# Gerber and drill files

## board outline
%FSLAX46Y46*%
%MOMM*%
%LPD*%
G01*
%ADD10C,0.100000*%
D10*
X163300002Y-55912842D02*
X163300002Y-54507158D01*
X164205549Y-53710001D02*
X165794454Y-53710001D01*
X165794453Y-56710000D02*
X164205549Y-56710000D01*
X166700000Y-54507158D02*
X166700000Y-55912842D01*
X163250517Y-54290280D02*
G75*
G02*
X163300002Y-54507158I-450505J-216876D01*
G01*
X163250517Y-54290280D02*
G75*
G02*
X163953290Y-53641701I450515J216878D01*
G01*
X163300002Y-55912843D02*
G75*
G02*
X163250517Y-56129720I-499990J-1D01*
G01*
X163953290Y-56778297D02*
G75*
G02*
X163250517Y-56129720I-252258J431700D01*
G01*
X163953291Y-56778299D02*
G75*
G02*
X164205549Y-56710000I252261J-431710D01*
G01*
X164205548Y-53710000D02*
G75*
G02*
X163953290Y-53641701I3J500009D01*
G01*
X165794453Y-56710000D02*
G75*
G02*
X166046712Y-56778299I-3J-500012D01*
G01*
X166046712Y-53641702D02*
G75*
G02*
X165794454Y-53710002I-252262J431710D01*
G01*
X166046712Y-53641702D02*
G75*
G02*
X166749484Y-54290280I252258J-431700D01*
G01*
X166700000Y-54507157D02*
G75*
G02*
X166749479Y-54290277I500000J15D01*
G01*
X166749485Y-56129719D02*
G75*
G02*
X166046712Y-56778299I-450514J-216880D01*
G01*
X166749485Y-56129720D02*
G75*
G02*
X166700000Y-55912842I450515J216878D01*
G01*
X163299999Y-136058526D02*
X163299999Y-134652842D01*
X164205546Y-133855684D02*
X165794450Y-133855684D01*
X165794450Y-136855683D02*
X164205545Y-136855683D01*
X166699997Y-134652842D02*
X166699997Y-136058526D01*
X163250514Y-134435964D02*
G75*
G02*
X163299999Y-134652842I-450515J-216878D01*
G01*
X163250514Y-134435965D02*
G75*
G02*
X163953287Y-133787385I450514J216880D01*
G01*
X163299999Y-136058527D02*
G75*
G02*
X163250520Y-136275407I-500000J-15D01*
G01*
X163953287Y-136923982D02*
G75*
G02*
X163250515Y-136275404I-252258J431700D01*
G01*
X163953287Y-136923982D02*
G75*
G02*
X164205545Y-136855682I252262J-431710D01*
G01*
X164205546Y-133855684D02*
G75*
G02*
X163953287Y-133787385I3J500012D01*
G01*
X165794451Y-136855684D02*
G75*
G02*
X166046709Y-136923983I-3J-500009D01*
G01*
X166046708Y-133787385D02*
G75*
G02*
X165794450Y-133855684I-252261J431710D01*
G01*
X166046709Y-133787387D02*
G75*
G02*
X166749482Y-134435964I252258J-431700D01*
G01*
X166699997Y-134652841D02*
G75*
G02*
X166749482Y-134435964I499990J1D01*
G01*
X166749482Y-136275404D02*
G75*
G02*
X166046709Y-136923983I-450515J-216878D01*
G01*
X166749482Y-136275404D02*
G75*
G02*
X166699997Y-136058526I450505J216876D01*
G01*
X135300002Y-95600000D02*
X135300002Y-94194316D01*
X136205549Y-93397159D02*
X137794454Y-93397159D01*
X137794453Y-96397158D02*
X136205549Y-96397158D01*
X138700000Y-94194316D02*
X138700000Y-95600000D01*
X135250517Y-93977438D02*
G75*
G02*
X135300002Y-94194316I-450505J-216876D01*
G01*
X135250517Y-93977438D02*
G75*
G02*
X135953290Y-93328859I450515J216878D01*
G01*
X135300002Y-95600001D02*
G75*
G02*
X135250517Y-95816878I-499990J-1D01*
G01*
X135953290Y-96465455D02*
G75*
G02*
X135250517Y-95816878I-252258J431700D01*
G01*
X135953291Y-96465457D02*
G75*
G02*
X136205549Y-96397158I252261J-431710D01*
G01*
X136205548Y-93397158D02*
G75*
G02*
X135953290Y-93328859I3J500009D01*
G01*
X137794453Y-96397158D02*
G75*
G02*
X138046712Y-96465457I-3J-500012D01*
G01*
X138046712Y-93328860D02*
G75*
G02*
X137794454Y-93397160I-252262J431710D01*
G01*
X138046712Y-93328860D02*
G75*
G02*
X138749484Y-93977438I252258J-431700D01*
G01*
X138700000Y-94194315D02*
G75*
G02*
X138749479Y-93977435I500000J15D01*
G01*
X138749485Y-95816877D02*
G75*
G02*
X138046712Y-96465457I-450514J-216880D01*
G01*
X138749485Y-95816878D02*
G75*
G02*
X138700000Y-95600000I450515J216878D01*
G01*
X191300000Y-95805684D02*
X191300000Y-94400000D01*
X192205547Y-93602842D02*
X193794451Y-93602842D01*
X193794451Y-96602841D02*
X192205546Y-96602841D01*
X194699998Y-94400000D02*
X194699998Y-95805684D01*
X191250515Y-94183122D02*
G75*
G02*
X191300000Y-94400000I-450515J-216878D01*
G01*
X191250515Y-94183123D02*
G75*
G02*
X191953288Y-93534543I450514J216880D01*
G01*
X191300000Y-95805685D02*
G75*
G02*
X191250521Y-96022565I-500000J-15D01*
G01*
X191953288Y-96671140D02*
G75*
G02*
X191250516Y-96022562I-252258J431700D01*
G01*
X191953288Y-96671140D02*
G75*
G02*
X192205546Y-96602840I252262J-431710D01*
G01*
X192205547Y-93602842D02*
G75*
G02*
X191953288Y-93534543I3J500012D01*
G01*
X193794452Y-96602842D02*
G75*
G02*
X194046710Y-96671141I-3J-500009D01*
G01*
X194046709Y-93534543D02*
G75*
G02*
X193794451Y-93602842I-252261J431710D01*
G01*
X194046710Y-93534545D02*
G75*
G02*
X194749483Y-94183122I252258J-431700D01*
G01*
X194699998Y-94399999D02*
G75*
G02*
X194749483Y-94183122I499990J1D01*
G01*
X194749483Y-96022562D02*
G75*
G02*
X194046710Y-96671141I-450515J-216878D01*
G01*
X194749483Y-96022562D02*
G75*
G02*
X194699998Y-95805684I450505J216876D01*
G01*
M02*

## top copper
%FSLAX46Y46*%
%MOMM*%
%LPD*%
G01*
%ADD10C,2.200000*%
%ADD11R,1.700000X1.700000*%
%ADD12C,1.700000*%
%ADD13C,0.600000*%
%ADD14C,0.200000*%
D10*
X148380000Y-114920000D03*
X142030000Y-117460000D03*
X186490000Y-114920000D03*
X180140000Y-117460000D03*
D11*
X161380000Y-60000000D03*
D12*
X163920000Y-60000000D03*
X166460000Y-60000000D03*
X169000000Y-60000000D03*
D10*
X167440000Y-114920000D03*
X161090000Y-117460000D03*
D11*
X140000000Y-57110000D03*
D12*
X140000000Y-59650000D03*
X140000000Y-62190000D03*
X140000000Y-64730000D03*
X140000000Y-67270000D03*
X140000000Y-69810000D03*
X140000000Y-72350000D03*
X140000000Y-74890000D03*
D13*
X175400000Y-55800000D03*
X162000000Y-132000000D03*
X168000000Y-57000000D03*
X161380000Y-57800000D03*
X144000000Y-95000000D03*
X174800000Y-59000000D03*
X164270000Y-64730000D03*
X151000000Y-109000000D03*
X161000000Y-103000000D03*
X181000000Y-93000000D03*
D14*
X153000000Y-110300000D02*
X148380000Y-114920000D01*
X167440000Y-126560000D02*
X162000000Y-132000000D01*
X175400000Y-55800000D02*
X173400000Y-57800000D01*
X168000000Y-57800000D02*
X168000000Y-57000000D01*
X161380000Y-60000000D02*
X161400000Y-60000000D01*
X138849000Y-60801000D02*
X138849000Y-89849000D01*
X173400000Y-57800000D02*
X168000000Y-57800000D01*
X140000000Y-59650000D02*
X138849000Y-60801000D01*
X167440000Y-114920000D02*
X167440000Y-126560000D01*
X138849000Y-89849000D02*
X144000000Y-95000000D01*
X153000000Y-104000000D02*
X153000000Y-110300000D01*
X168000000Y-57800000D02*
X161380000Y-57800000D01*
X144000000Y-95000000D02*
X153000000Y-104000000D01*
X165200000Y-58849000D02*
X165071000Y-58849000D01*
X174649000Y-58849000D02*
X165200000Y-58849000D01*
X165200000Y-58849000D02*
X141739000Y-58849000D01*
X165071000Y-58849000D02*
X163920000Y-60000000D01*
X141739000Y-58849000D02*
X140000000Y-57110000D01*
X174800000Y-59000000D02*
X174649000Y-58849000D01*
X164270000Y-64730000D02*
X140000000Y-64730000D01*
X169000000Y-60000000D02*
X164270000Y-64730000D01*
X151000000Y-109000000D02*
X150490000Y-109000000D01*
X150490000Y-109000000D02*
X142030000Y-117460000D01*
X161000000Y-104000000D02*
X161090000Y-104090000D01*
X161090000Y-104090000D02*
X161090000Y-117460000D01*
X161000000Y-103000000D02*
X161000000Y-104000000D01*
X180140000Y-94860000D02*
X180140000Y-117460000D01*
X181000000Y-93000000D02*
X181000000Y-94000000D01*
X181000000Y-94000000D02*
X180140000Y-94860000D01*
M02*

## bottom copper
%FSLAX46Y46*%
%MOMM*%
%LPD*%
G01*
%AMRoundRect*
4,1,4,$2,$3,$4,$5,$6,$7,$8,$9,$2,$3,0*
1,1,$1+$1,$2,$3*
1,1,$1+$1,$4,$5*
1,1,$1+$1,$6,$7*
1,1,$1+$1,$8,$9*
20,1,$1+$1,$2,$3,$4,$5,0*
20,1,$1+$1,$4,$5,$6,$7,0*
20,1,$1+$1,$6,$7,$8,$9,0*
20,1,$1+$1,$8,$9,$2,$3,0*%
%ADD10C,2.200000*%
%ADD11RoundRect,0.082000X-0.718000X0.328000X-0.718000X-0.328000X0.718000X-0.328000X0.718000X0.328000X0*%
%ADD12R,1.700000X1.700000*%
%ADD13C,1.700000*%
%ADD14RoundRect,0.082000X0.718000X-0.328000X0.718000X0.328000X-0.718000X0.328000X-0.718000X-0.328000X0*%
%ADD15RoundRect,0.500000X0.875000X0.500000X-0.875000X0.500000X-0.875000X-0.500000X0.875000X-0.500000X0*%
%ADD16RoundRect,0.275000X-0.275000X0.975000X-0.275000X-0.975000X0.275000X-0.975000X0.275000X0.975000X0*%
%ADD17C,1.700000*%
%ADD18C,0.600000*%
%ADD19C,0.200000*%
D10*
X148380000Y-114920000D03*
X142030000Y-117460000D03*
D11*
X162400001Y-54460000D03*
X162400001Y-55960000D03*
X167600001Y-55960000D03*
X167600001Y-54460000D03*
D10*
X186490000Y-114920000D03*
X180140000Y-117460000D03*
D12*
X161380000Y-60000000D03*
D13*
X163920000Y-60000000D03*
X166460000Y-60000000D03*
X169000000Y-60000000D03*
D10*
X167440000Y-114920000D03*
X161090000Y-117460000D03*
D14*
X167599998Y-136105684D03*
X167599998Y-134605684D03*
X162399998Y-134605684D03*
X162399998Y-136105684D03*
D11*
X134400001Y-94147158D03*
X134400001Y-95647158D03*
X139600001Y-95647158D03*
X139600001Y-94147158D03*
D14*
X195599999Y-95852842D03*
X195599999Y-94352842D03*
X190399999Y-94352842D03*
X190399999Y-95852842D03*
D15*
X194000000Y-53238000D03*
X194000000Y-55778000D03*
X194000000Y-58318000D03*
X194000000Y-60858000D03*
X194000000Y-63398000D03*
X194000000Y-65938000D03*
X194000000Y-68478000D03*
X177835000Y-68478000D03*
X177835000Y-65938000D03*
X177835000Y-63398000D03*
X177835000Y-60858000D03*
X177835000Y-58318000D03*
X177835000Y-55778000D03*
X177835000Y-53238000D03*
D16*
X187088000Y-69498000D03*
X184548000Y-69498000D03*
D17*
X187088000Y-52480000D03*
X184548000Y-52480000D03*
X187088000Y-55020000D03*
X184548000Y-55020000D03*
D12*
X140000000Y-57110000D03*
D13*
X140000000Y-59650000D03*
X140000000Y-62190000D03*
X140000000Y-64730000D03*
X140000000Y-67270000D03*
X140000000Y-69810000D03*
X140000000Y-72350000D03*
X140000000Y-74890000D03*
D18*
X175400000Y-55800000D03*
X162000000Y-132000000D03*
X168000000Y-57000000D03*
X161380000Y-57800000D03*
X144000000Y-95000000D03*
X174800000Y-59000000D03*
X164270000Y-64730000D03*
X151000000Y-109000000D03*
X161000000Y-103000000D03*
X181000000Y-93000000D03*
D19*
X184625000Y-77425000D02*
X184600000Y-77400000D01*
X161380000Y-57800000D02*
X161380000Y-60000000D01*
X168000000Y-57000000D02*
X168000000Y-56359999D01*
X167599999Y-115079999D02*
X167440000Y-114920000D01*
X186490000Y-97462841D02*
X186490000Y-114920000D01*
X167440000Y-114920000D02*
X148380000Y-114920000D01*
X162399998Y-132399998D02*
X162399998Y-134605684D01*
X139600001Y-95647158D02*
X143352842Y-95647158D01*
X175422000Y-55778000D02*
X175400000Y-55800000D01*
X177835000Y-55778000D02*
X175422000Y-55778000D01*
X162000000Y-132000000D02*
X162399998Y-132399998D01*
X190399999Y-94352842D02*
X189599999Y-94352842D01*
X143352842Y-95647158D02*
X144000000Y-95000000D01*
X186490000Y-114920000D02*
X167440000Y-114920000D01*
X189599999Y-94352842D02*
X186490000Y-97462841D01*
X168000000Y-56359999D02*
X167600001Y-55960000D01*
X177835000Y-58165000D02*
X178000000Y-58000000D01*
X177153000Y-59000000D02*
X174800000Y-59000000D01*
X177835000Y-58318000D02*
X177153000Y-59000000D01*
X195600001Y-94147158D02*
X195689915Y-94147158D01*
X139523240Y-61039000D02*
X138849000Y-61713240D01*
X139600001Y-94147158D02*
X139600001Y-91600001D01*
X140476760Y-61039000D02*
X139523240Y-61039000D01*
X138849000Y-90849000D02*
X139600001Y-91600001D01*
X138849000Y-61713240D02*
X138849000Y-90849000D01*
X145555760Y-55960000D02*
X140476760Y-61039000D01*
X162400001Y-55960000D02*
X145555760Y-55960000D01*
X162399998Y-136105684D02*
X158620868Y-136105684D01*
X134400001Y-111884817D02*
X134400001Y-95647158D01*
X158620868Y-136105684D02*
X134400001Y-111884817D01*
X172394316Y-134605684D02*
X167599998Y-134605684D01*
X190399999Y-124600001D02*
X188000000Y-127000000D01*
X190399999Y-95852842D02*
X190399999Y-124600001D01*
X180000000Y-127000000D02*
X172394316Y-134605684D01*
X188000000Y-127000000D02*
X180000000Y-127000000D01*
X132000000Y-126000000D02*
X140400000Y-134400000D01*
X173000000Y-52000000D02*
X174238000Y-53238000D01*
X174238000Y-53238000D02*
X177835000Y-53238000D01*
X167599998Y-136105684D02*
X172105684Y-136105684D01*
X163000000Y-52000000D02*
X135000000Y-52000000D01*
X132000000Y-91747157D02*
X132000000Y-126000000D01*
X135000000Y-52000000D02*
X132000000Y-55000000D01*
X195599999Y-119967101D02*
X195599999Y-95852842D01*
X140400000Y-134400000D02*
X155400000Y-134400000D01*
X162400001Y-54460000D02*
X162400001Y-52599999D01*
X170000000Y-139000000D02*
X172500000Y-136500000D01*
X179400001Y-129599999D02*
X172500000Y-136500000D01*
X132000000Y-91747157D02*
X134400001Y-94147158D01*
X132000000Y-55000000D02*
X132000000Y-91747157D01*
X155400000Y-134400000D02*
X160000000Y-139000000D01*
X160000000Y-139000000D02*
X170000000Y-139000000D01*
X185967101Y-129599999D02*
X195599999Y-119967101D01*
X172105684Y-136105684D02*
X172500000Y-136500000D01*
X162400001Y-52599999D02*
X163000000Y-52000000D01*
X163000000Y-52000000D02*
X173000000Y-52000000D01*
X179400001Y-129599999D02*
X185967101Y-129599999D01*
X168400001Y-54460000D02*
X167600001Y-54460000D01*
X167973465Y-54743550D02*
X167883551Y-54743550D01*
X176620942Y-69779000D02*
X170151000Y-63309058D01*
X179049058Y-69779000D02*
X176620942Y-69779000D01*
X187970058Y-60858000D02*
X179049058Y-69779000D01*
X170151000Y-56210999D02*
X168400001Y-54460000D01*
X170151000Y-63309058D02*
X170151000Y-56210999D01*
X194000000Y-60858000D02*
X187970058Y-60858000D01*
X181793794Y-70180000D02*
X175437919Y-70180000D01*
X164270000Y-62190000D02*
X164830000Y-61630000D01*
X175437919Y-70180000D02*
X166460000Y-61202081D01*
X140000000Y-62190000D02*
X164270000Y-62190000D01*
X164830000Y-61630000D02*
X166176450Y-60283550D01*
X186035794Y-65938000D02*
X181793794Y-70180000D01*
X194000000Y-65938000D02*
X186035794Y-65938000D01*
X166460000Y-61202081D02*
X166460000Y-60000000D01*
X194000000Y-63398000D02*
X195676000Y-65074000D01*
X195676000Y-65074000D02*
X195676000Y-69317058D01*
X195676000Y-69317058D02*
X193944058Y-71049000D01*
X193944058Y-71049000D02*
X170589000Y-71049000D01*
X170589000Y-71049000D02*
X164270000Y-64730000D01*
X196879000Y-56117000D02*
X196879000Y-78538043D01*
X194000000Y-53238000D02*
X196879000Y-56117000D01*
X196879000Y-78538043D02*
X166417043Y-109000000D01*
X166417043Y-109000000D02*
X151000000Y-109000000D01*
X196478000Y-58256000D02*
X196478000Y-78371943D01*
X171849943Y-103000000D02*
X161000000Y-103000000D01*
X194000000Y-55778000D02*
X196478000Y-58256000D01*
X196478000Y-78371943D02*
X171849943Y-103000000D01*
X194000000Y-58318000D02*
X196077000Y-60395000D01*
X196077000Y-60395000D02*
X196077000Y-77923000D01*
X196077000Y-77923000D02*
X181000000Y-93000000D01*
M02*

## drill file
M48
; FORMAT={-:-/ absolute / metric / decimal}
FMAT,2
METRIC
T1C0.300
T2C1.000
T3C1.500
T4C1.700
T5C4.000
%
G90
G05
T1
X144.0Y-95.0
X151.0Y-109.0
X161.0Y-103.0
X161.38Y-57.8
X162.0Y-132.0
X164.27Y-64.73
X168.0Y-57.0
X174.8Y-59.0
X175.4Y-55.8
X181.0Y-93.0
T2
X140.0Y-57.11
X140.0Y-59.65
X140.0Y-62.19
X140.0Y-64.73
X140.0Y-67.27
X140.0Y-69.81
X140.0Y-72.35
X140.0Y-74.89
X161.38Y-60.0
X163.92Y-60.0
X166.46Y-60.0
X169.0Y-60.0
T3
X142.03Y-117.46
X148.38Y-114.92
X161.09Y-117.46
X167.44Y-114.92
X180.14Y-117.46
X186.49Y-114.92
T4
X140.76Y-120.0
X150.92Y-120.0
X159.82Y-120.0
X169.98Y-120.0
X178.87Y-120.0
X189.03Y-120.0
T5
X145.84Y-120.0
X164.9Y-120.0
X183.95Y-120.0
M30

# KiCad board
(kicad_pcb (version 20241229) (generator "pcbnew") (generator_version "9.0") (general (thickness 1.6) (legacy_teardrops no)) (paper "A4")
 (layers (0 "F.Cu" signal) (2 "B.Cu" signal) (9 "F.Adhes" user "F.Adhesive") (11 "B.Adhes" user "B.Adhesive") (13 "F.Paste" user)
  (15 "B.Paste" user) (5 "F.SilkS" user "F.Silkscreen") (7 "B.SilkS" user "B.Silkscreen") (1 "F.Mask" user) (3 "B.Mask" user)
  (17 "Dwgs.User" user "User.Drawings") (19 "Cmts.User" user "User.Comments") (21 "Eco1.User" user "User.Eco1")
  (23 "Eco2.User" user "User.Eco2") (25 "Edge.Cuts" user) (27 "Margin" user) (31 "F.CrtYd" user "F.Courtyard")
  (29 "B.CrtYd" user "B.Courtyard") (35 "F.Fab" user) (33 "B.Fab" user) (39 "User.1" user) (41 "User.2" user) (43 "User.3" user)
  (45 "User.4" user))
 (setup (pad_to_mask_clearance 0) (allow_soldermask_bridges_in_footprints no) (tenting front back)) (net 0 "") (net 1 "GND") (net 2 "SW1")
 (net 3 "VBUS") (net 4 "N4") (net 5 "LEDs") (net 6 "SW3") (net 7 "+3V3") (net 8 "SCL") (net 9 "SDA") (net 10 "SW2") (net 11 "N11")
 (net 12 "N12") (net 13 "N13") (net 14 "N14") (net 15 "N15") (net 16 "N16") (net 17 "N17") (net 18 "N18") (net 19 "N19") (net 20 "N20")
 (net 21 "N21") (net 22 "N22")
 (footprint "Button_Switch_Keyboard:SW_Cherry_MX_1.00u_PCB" (layer "F.Cu") (at 148.38 114.92)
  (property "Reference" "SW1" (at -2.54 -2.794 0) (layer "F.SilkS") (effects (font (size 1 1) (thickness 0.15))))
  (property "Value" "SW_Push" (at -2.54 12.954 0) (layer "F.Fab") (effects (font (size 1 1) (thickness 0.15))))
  (pad "" np_thru_hole circle (at -7.62 5.08) (size 1.7 1.7) (drill 1.7) (layers "*.Cu" "*.Mask"))
  (pad "" np_thru_hole circle (at -2.54 5.08) (size 4 4) (drill 4) (layers "*.Cu" "*.Mask"))
  (pad "" np_thru_hole circle (at 2.54 5.08) (size 1.7 1.7) (drill 1.7) (layers "*.Cu" "*.Mask"))
  (pad "1" thru_hole circle (at 0 0) (size 2.2 2.2) (drill 1.5) (layers "*.Cu" "*.Mask") (remove_unused_layers no) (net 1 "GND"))
  (pad "2" thru_hole circle (at -6.35 2.54) (size 2.2 2.2) (drill 1.5) (layers "*.Cu" "*.Mask") (remove_unused_layers no) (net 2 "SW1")))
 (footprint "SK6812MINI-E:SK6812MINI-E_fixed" (layer "F.Cu") (at 165 55.312842)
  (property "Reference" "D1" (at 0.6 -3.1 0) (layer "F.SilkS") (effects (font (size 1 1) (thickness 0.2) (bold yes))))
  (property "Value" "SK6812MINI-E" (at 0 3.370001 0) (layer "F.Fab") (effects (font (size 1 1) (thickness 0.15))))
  (fp_line (start -1.699998 0.6) (end -1.699998 -0.805684) (stroke (width 0.1) (type solid)) (layer "Edge.Cuts"))
  (fp_line (start -0.794451 -1.602841) (end 0.794454 -1.602841) (stroke (width 0.1) (type solid)) (layer "Edge.Cuts"))
  (fp_line (start 0.794453 1.397158) (end -0.794451 1.397158) (stroke (width 0.1) (type solid)) (layer "Edge.Cuts"))
  (fp_line (start 1.7 -0.805684) (end 1.7 0.6) (stroke (width 0.1) (type solid)) (layer "Edge.Cuts"))
  (fp_arc (start -1.749483 -1.022562) (mid -1.712526 -0.91691) (end -1.699998 -0.805684) (stroke (width 0.1) (type solid))
   (layer "Edge.Cuts"))
  (fp_arc (start -1.749483 -1.022562) (mid -1.63807 -1.606877) (end -1.04671 -1.671141) (stroke (width 0.1) (type solid))
   (layer "Edge.Cuts"))
  (fp_arc (start -1.699998 0.600001) (mid -1.712526 0.711226) (end -1.749483 0.816878) (stroke (width 0.1) (type solid)) (layer "Edge.Cuts"))
  (fp_arc (start -1.04671 1.465455) (mid -1.638069 1.401192) (end -1.749483 0.816878) (stroke (width 0.1) (type solid)) (layer "Edge.Cuts"))
  (fp_arc (start -1.046709 1.465457) (mid -0.925121 1.414535) (end -0.794451 1.397158) (stroke (width 0.1) (type solid)) (layer "Edge.Cuts"))
  (fp_arc (start -0.794452 -1.602842) (mid -0.925122 -1.620219) (end -1.04671 -1.671141) (stroke (width 0.1) (type solid))
   (layer "Edge.Cuts"))
  (fp_arc (start 0.794453 1.397158) (mid 0.925124 1.414535) (end 1.046712 1.465457) (stroke (width 0.1) (type solid)) (layer "Edge.Cuts"))
  (fp_arc (start 1.046712 -1.67114) (mid 0.925124 -1.620218) (end 0.794454 -1.602841) (stroke (width 0.1) (type solid)) (layer "Edge.Cuts"))
  (fp_arc (start 1.046712 -1.67114) (mid 1.638072 -1.606876) (end 1.749485 -1.022562) (stroke (width 0.1) (type solid)) (layer "Edge.Cuts"))
  (fp_arc (start 1.7 -0.805685) (mid 1.712528 -0.91691) (end 1.749485 -1.022562) (stroke (width 0.1) (type solid)) (layer "Edge.Cuts"))
  (fp_arc (start 1.749485 0.816877) (mid 1.638073 1.401193) (end 1.046712 1.465457) (stroke (width 0.1) (type solid)) (layer "Edge.Cuts"))
  (fp_arc (start 1.749485 0.816878) (mid 1.712528 0.711226) (end 1.7 0.6) (stroke (width 0.1) (type solid)) (layer "Edge.Cuts"))
  (pad "1" smd roundrect (at -2.599999 -0.852842 270) (size 0.82 1.6) (layers "B.Cu" "B.Mask" "B.Paste") (roundrect_rratio 0.1)
   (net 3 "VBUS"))
  (pad "2" smd roundrect (at -2.599999 0.647158 270) (size 0.82 1.6) (layers "B.Cu" "B.Mask" "B.Paste") (roundrect_rratio 0.1) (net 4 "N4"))
  (pad "3" smd roundrect (at 2.600001 0.647158 270) (size 0.82 1.6) (layers "B.Cu" "B.Mask" "B.Paste") (roundrect_rratio 0.1) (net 1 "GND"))
  (pad "4" smd roundrect (at 2.600001 -0.852842 270) (size 0.82 1.6) (layers "B.Cu" "B.Mask" "B.Paste") (roundrect_rratio 0.1)
   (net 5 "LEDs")))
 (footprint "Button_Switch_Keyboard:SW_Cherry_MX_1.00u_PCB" (layer "F.Cu") (at 186.49 114.92)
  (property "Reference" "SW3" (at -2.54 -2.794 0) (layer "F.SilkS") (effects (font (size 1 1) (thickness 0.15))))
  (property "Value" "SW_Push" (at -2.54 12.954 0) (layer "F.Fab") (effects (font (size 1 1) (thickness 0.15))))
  (pad "" np_thru_hole circle (at -7.62 5.08) (size 1.7 1.7) (drill 1.7) (layers "*.Cu" "*.Mask"))
  (pad "" np_thru_hole circle (at -2.54 5.08) (size 4 4) (drill 4) (layers "*.Cu" "*.Mask"))
  (pad "" np_thru_hole circle (at 2.54 5.08) (size 1.7 1.7) (drill 1.7) (layers "*.Cu" "*.Mask"))
  (pad "1" thru_hole circle (at 0 0) (size 2.2 2.2) (drill 1.5) (layers "*.Cu" "*.Mask") (remove_unused_layers no) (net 1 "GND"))
  (pad "2" thru_hole circle (at -6.35 2.54) (size 2.2 2.2) (drill 1.5) (layers "*.Cu" "*.Mask") (remove_unused_layers no) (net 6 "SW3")))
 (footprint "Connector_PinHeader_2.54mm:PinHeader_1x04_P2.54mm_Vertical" (layer "F.Cu") (at 161.38 60 90)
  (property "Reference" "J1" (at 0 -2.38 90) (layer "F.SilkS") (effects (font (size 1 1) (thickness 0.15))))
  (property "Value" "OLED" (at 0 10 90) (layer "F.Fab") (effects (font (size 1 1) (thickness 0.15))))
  (pad "1" thru_hole rect (at 0 0 90) (size 1.7 1.7) (drill 1) (layers "*.Cu" "*.Mask") (remove_unused_layers no) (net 1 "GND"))
  (pad "2" thru_hole circle (at 0 2.54 90) (size 1.7 1.7) (drill 1) (layers "*.Cu" "*.Mask") (remove_unused_layers no) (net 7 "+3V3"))
  (pad "3" thru_hole circle (at 0 5.08 90) (size 1.7 1.7) (drill 1) (layers "*.Cu" "*.Mask") (remove_unused_layers no) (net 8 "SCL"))
  (pad "4" thru_hole circle (at 0 7.62 90) (size 1.7 1.7) (drill 1) (layers "*.Cu" "*.Mask") (remove_unused_layers no) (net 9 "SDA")))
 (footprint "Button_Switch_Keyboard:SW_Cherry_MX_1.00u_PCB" (layer "F.Cu") (at 167.44 114.92)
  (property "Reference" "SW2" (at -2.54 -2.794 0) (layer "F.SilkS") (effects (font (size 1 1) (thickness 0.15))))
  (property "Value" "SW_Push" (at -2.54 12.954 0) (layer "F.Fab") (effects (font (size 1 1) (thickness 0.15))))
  (pad "" np_thru_hole circle (at -7.62 5.08) (size 1.7 1.7) (drill 1.7) (layers "*.Cu" "*.Mask"))
  (pad "" np_thru_hole circle (at -2.54 5.08) (size 4 4) (drill 4) (layers "*.Cu" "*.Mask"))
  (pad "" np_thru_hole circle (at 2.54 5.08) (size 1.7 1.7) (drill 1.7) (layers "*.Cu" "*.Mask"))
  (pad "1" thru_hole circle (at 0 0) (size 2.2 2.2) (drill 1.5) (layers "*.Cu" "*.Mask") (remove_unused_layers no) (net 1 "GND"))
  (pad "2" thru_hole circle (at -6.35 2.54) (size 2.2 2.2) (drill 1.5) (layers "*.Cu" "*.Mask") (remove_unused_layers no) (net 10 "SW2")))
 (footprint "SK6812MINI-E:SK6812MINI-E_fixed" (layer "F.Cu") (at 164.999999 135.252842 180)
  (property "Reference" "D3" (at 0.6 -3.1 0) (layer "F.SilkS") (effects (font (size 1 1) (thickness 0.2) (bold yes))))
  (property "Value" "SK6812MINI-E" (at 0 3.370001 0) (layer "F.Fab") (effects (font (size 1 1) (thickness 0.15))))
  (fp_line (start 1.7 -0.805684) (end 1.7 0.6) (stroke (width 0.1) (type solid)) (layer "Edge.Cuts"))
  (fp_line (start 0.794453 1.397158) (end -0.794451 1.397158) (stroke (width 0.1) (type solid)) (layer "Edge.Cuts"))
  (fp_line (start -0.794451 -1.602841) (end 0.794454 -1.602841) (stroke (width 0.1) (type solid)) (layer "Edge.Cuts"))
  (fp_line (start -1.699998 0.6) (end -1.699998 -0.805684) (stroke (width 0.1) (type solid)) (layer "Edge.Cuts"))
  (fp_arc (start 1.749485 0.816878) (mid 1.712528 0.711226) (end 1.7 0.6) (stroke (width 0.1) (type solid)) (layer "Edge.Cuts"))
  (fp_arc (start 1.749485 0.816877) (mid 1.638073 1.401193) (end 1.046712 1.465457) (stroke (width 0.1) (type solid)) (layer "Edge.Cuts"))
  (fp_arc (start 1.7 -0.805685) (mid 1.712528 -0.91691) (end 1.749485 -1.022562) (stroke (width 0.1) (type solid)) (layer "Edge.Cuts"))
  (fp_arc (start 1.046712 -1.67114) (mid 1.638072 -1.606876) (end 1.749485 -1.022562) (stroke (width 0.1) (type solid)) (layer "Edge.Cuts"))
  (fp_arc (start 1.046712 -1.67114) (mid 0.925124 -1.620218) (end 0.794454 -1.602841) (stroke (width 0.1) (type solid)) (layer "Edge.Cuts"))
  (fp_arc (start 0.794453 1.397158) (mid 0.925124 1.414535) (end 1.046712 1.465457) (stroke (width 0.1) (type solid)) (layer "Edge.Cuts"))
  (fp_arc (start -0.794452 -1.602842) (mid -0.925122 -1.620219) (end -1.04671 -1.671141) (stroke (width 0.1) (type solid))
   (layer "Edge.Cuts"))
  (fp_arc (start -1.046709 1.465457) (mid -0.925121 1.414535) (end -0.794451 1.397158) (stroke (width 0.1) (type solid)) (layer "Edge.Cuts"))
  (fp_arc (start -1.04671 1.465455) (mid -1.638069 1.401192) (end -1.749483 0.816878) (stroke (width 0.1) (type solid)) (layer "Edge.Cuts"))
  (fp_arc (start -1.699998 0.600001) (mid -1.712526 0.711226) (end -1.749483 0.816878) (stroke (width 0.1) (type solid)) (layer "Edge.Cuts"))
  (fp_arc (start -1.749483 -1.022562) (mid -1.63807 -1.606877) (end -1.04671 -1.671141) (stroke (width 0.1) (type solid))
   (layer "Edge.Cuts"))
  (fp_arc (start -1.749483 -1.022562) (mid -1.712526 -0.91691) (end -1.699998 -0.805684) (stroke (width 0.1) (type solid))
   (layer "Edge.Cuts"))
  (pad "1" smd roundrect (at -2.599999 -0.852842 90) (size 0.82 1.6) (layers "B.Cu" "B.Mask" "B.Paste") (roundrect_rratio 0.1)
   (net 3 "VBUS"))
  (pad "2" smd roundrect (at -2.599999 0.647158 90) (size 0.82 1.6) (layers "B.Cu" "B.Mask" "B.Paste") (roundrect_rratio 0.1) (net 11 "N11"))
  (pad "3" smd roundrect (at 2.600001 0.647158 90) (size 0.82 1.6) (layers "B.Cu" "B.Mask" "B.Paste") (roundrect_rratio 0.1) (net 1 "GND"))
  (pad "4" smd roundrect (at 2.600001 -0.852842 90) (size 0.82 1.6) (layers "B.Cu" "B.Mask" "B.Paste") (roundrect_rratio 0.1) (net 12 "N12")))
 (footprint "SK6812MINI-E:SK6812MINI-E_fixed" (layer "F.Cu") (at 137 95)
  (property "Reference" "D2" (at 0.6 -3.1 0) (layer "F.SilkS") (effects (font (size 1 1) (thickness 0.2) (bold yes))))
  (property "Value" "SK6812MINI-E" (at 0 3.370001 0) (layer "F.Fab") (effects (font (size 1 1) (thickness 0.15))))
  (fp_line (start -1.699998 0.6) (end -1.699998 -0.805684) (stroke (width 0.1) (type solid)) (layer "Edge.Cuts"))
  (fp_line (start -0.794451 -1.602841) (end 0.794454 -1.602841) (stroke (width 0.1) (type solid)) (layer "Edge.Cuts"))
  (fp_line (start 0.794453 1.397158) (end -0.794451 1.397158) (stroke (width 0.1) (type solid)) (layer "Edge.Cuts"))
  (fp_line (start 1.7 -0.805684) (end 1.7 0.6) (stroke (width 0.1) (type solid)) (layer "Edge.Cuts"))
  (fp_arc (start -1.749483 -1.022562) (mid -1.712526 -0.91691) (end -1.699998 -0.805684) (stroke (width 0.1) (type solid))
   (layer "Edge.Cuts"))
  (fp_arc (start -1.749483 -1.022562) (mid -1.63807 -1.606877) (end -1.04671 -1.671141) (stroke (width 0.1) (type solid))
   (layer "Edge.Cuts"))
  (fp_arc (start -1.699998 0.600001) (mid -1.712526 0.711226) (end -1.749483 0.816878) (stroke (width 0.1) (type solid)) (layer "Edge.Cuts"))
  (fp_arc (start -1.04671 1.465455) (mid -1.638069 1.401192) (end -1.749483 0.816878) (stroke (width 0.1) (type solid)) (layer "Edge.Cuts"))
  (fp_arc (start -1.046709 1.465457) (mid -0.925121 1.414535) (end -0.794451 1.397158) (stroke (width 0.1) (type solid)) (layer "Edge.Cuts"))
  (fp_arc (start -0.794452 -1.602842) (mid -0.925122 -1.620219) (end -1.04671 -1.671141) (stroke (width 0.1) (type solid))
   (layer "Edge.Cuts"))
  (fp_arc (start 0.794453 1.397158) (mid 0.925124 1.414535) (end 1.046712 1.465457) (stroke (width 0.1) (type solid)) (layer "Edge.Cuts"))
  (fp_arc (start 1.046712 -1.67114) (mid 0.925124 -1.620218) (end 0.794454 -1.602841) (stroke (width 0.1) (type solid)) (layer "Edge.Cuts"))
  (fp_arc (start 1.046712 -1.67114) (mid 1.638072 -1.606876) (end 1.749485 -1.022562) (stroke (width 0.1) (type solid)) (layer "Edge.Cuts"))
  (fp_arc (start 1.7 -0.805685) (mid 1.712528 -0.91691) (end 1.749485 -1.022562) (stroke (width 0.1) (type solid)) (layer "Edge.Cuts"))
  (fp_arc (start 1.749485 0.816877) (mid 1.638073 1.401193) (end 1.046712 1.465457) (stroke (width 0.1) (type solid)) (layer "Edge.Cuts"))
  (fp_arc (start 1.749485 0.816878) (mid 1.712528 0.711226) (end 1.7 0.6) (stroke (width 0.1) (type solid)) (layer "Edge.Cuts"))
  (pad "1" smd roundrect (at -2.599999 -0.852842 270) (size 0.82 1.6) (layers "B.Cu" "B.Mask" "B.Paste") (roundrect_rratio 0.1)
   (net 3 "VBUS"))
  (pad "2" smd roundrect (at -2.599999 0.647158 270) (size 0.82 1.6) (layers "B.Cu" "B.Mask" "B.Paste") (roundrect_rratio 0.1)
   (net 12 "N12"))
  (pad "3" smd roundrect (at 2.600001 0.647158 270) (size 0.82 1.6) (layers "B.Cu" "B.Mask" "B.Paste") (roundrect_rratio 0.1) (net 1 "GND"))
  (pad "4" smd roundrect (at 2.600001 -0.852842 270) (size 0.82 1.6) (layers "B.Cu" "B.Mask" "B.Paste") (roundrect_rratio 0.1) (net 4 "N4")))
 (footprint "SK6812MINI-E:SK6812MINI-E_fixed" (layer "F.Cu") (at 193 95 180)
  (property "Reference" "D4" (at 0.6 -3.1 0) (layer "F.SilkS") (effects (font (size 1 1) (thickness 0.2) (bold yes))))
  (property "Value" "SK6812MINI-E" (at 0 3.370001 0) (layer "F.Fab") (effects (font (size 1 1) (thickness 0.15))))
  (fp_line (start 1.7 -0.805684) (end 1.7 0.6) (stroke (width 0.1) (type solid)) (layer "Edge.Cuts"))
  (fp_line (start 0.794453 1.397158) (end -0.794451 1.397158) (stroke (width 0.1) (type solid)) (layer "Edge.Cuts"))
  (fp_line (start -0.794451 -1.602841) (end 0.794454 -1.602841) (stroke (width 0.1) (type solid)) (layer "Edge.Cuts"))
  (fp_line (start -1.699998 0.6) (end -1.699998 -0.805684) (stroke (width 0.1) (type solid)) (layer "Edge.Cuts"))
  (fp_arc (start 1.749485 0.816878) (mid 1.712528 0.711226) (end 1.7 0.6) (stroke (width 0.1) (type solid)) (layer "Edge.Cuts"))
  (fp_arc (start 1.749485 0.816877) (mid 1.638073 1.401193) (end 1.046712 1.465457) (stroke (width 0.1) (type solid)) (layer "Edge.Cuts"))
  (fp_arc (start 1.7 -0.805685) (mid 1.712528 -0.91691) (end 1.749485 -1.022562) (stroke (width 0.1) (type solid)) (layer "Edge.Cuts"))
  (fp_arc (start 1.046712 -1.67114) (mid 1.638072 -1.606876) (end 1.749485 -1.022562) (stroke (width 0.1) (type solid)) (layer "Edge.Cuts"))
  (fp_arc (start 1.046712 -1.67114) (mid 0.925124 -1.620218) (end 0.794454 -1.602841) (stroke (width 0.1) (type solid)) (layer "Edge.Cuts"))
  (fp_arc (start 0.794453 1.397158) (mid 0.925124 1.414535) (end 1.046712 1.465457) (stroke (width 0.1) (type solid)) (layer "Edge.Cuts"))
  (fp_arc (start -0.794452 -1.602842) (mid -0.925122 -1.620219) (end -1.04671 -1.671141) (stroke (width 0.1) (type solid))
   (layer "Edge.Cuts"))
  (fp_arc (start -1.046709 1.465457) (mid -0.925121 1.414535) (end -0.794451 1.397158) (stroke (width 0.1) (type solid)) (layer "Edge.Cuts"))
  (fp_arc (start -1.04671 1.465455) (mid -1.638069 1.401192) (end -1.749483 0.816878) (stroke (width 0.1) (type solid)) (layer "Edge.Cuts"))
  (fp_arc (start -1.699998 0.600001) (mid -1.712526 0.711226) (end -1.749483 0.816878) (stroke (width 0.1) (type solid)) (layer "Edge.Cuts"))
  (fp_arc (start -1.749483 -1.022562) (mid -1.63807 -1.606877) (end -1.04671 -1.671141) (stroke (width 0.1) (type solid))
   (layer "Edge.Cuts"))
  (fp_arc (start -1.749483 -1.022562) (mid -1.712526 -0.91691) (end -1.699998 -0.805684) (stroke (width 0.1) (type solid))
   (layer "Edge.Cuts"))
  (pad "1" smd roundrect (at -2.599999 -0.852842 90) (size 0.82 1.6) (layers "B.Cu" "B.Mask" "B.Paste") (roundrect_rratio 0.1)
   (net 3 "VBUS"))
  (pad "2" smd roundrect (at -2.599999 0.647158 90) (size 0.82 1.6) (layers "B.Cu" "B.Mask" "B.Paste") (roundrect_rratio 0.1) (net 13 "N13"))
  (pad "3" smd roundrect (at 2.600001 0.647158 90) (size 0.82 1.6) (layers "B.Cu" "B.Mask" "B.Paste") (roundrect_rratio 0.1) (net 1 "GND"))
  (pad "4" smd roundrect (at 2.600001 -0.852842 90) (size 0.82 1.6) (layers "B.Cu" "B.Mask" "B.Paste") (roundrect_rratio 0.1) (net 11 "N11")))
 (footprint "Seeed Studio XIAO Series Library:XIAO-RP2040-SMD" (layer "B.Cu") (at 186 60.858 180)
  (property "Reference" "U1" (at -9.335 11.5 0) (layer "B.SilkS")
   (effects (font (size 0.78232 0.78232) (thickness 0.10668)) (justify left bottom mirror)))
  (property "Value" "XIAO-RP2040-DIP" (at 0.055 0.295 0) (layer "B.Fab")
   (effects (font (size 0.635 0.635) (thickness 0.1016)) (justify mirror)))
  (pad "1" smd roundrect (at -8 7.62 180) (size 2.75 2) (layers "B.Cu" "B.Mask" "B.Paste") (roundrect_rratio 0.25) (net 2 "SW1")
   (solder_mask_margin 0.0508) (thermal_bridge_angle 45))
  (pad "2" smd roundrect (at -8 5.08 180) (size 2.75 2) (layers "B.Cu" "B.Mask" "B.Paste") (roundrect_rratio 0.25) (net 10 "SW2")
   (solder_mask_margin 0.0508) (thermal_bridge_angle 45))
  (pad "3" smd roundrect (at -8 2.54 180) (size 2.75 2) (layers "B.Cu" "B.Mask" "B.Paste") (roundrect_rratio 0.25) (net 6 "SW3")
   (solder_mask_margin 0.0508) (thermal_bridge_angle 45))
  (pad "4" smd roundrect (at -8 0 180) (size 2.75 2) (layers "B.Cu" "B.Mask" "B.Paste") (roundrect_rratio 0.25) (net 5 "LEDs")
   (solder_mask_margin 0.0508) (thermal_bridge_angle 45))
  (pad "5" smd roundrect (at -8 -2.54 180) (size 2.75 2) (layers "B.Cu" "B.Mask" "B.Paste") (roundrect_rratio 0.25) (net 9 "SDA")
   (solder_mask_margin 0.0508) (thermal_bridge_angle 45))
  (pad "6" smd roundrect (at -8 -5.08 180) (size 2.75 2) (layers "B.Cu" "B.Mask" "B.Paste") (roundrect_rratio 0.25) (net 8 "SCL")
   (solder_mask_margin 0.0508) (thermal_bridge_angle 45))
  (pad "7" smd roundrect (at -8 -7.62 180) (size 2.75 2) (layers "B.Cu" "B.Mask" "B.Paste") (roundrect_rratio 0.25) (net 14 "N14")
   (solder_mask_margin 0.0508) (thermal_bridge_angle 45))
  (pad "8" smd roundrect (at 8.165 -7.62 180) (size 2.75 2) (layers "B.Cu" "B.Mask" "B.Paste") (roundrect_rratio 0.25) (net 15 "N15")
   (solder_mask_margin 0.0508) (thermal_bridge_angle 45))
  (pad "9" smd roundrect (at 8.165 -5.08 180) (size 2.75 2) (layers "B.Cu" "B.Mask" "B.Paste") (roundrect_rratio 0.25) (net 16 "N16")
   (solder_mask_margin 0.0508) (thermal_bridge_angle 45))
  (pad "10" smd roundrect (at 8.165 -2.54 180) (size 2.75 2) (layers "B.Cu" "B.Mask" "B.Paste") (roundrect_rratio 0.25) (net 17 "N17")
   (solder_mask_margin 0.0508) (thermal_bridge_angle 45))
  (pad "11" smd roundrect (at 8.165 0 180) (size 2.75 2) (layers "B.Cu" "B.Mask" "B.Paste") (roundrect_rratio 0.25) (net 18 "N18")
   (solder_mask_margin 0.0508) (thermal_bridge_angle 45))
  (pad "12" smd roundrect (at 8.165 2.54 180) (size 2.75 2) (layers "B.Cu" "B.Mask" "B.Paste") (roundrect_rratio 0.25) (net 7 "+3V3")
   (solder_mask_margin 0.0508) (thermal_bridge_angle 45))
  (pad "13" smd roundrect (at 8.165 5.08 180) (size 2.75 2) (layers "B.Cu" "B.Mask" "B.Paste") (roundrect_rratio 0.25) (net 1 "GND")
   (solder_mask_margin 0.0508) (thermal_bridge_angle 45))
  (pad "14" smd roundrect (at 8.165 7.62 180) (size 2.75 2) (layers "B.Cu" "B.Mask" "B.Paste") (roundrect_rratio 0.25) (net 3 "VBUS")
   (solder_mask_margin 0.0508) (thermal_bridge_angle 45))
  (pad "15" smd roundrect (at -1.088 -8.64 270) (size 2.5 1.1) (layers "B.Cu" "B.Mask" "B.Paste") (roundrect_rratio 0.25)
   (thermal_bridge_angle 45))
  (pad "16" smd roundrect (at 1.452 -8.64 270) (size 2.5 1.1) (layers "B.Cu" "B.Mask" "B.Paste") (roundrect_rratio 0.25)
   (thermal_bridge_angle 45))
  (pad "17" smd circle (at -1.088 8.378 180) (size 1.7 1.7) (layers "B.Cu" "B.Mask" "B.Paste"))
  (pad "18" smd circle (at 1.452 8.378 180) (size 1.7 1.7) (layers "B.Cu" "B.Mask" "B.Paste"))
  (pad "19" smd circle (at -1.088 5.838 180) (size 1.7 1.7) (layers "B.Cu" "B.Mask" "B.Paste"))
  (pad "20" smd circle (at 1.452 5.838 180) (size 1.7 1.7) (layers "B.Cu" "B.Mask" "B.Paste")))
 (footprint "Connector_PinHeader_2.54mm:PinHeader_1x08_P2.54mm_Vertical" (layer "B.Cu") (at 140 57.11 180)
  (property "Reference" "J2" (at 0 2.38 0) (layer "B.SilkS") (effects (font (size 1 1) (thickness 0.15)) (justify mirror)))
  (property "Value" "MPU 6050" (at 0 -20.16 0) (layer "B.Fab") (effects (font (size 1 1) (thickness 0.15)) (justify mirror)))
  (pad "1" thru_hole rect (at 0 0 180) (size 1.7 1.7) (drill 1) (layers "*.Cu" "*.Mask") (remove_unused_layers no) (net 7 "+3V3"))
  (pad "2" thru_hole circle (at 0 -2.54 180) (size 1.7 1.7) (drill 1) (layers "*.Cu" "*.Mask") (remove_unused_layers no) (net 1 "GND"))
  (pad "3" thru_hole circle (at 0 -5.08 180) (size 1.7 1.7) (drill 1) (layers "*.Cu" "*.Mask") (remove_unused_layers no) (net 8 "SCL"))
  (pad "4" thru_hole circle (at 0 -7.62 180) (size 1.7 1.7) (drill 1) (layers "*.Cu" "*.Mask") (remove_unused_layers no) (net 9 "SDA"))
  (pad "5" thru_hole circle (at 0 -10.16 180) (size 1.7 1.7) (drill 1) (layers "*.Cu" "*.Mask") (remove_unused_layers no) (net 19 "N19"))
  (pad "6" thru_hole circle (at 0 -12.7 180) (size 1.7 1.7) (drill 1) (layers "*.Cu" "*.Mask") (remove_unused_layers no) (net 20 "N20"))
  (pad "7" thru_hole circle (at 0 -15.24 180) (size 1.7 1.7) (drill 1) (layers "*.Cu" "*.Mask") (remove_unused_layers no) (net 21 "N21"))
  (pad "8" thru_hole circle (at 0 -17.78 180) (size 1.7 1.7) (drill 1) (layers "*.Cu" "*.Mask") (remove_unused_layers no) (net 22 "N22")))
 (segment (start 184.625 77.425) (end 184.6 77.4) (width 0.2) (layer "B.Cu") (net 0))
 (segment (start 153 110.3) (end 148.38 114.92) (width 0.2) (layer "F.Cu") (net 1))
 (segment (start 167.44 126.56) (end 162 132) (width 0.2) (layer "F.Cu") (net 1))
 (segment (start 175.4 55.8) (end 173.4 57.8) (width 0.2) (layer "F.Cu") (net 1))
 (segment (start 168 57.8) (end 168 57) (width 0.2) (layer "F.Cu") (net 1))
 (segment (start 161.38 60) (end 161.4 60) (width 0.2) (layer "F.Cu") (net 1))
 (segment (start 138.849 60.801) (end 138.849 89.849) (width 0.2) (layer "F.Cu") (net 1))
 (segment (start 173.4 57.8) (end 168 57.8) (width 0.2) (layer "F.Cu") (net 1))
 (segment (start 140 59.65) (end 138.849 60.801) (width 0.2) (layer "F.Cu") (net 1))
 (segment (start 167.44 114.92) (end 167.44 126.56) (width 0.2) (layer "F.Cu") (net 1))
 (segment (start 138.849 89.849) (end 144 95) (width 0.2) (layer "F.Cu") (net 1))
 (segment (start 153 104) (end 153 110.3) (width 0.2) (layer "F.Cu") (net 1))
 (segment (start 168 57.8) (end 161.38 57.8) (width 0.2) (layer "F.Cu") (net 1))
 (segment (start 144 95) (end 153 104) (width 0.2) (layer "F.Cu") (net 1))
 (via (at 175.4 55.8) (size 0.6) (drill 0.3) (layers "F.Cu" "B.Cu") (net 1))
 (via (at 162 132) (size 0.6) (drill 0.3) (layers "F.Cu" "B.Cu") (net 1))
 (via (at 168 57) (size 0.6) (drill 0.3) (layers "F.Cu" "B.Cu") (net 1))
 (via (at 161.38 57.8) (size 0.6) (drill 0.3) (layers "F.Cu" "B.Cu") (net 1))
 (via (at 144 95) (size 0.6) (drill 0.3) (layers "F.Cu" "B.Cu") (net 1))
 (segment (start 161.38 57.8) (end 161.38 60) (width 0.2) (layer "B.Cu") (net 1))
 (segment (start 168 57) (end 168 56.359999) (width 0.2) (layer "B.Cu") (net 1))
 (segment (start 167.599999 115.079999) (end 167.44 114.92) (width 0.2) (layer "B.Cu") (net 1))
 (segment (start 186.49 97.462841) (end 186.49 114.92) (width 0.2) (layer "B.Cu") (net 1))
 (segment (start 167.44 114.92) (end 148.38 114.92) (width 0.2) (layer "B.Cu") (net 1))
 (segment (start 162.399998 132.399998) (end 162.399998 134.605684) (width 0.2) (layer "B.Cu") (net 1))
 (segment (start 139.600001 95.647158) (end 143.352842 95.647158) (width 0.2) (layer "B.Cu") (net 1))
 (segment (start 175.422 55.778) (end 175.4 55.8) (width 0.2) (layer "B.Cu") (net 1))
 (segment (start 177.835 55.778) (end 175.422 55.778) (width 0.2) (layer "B.Cu") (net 1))
 (segment (start 162 132) (end 162.399998 132.399998) (width 0.2) (layer "B.Cu") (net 1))
 (segment (start 190.399999 94.352842) (end 189.599999 94.352842) (width 0.2) (layer "B.Cu") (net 1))
 (segment (start 143.352842 95.647158) (end 144 95) (width 0.2) (layer "B.Cu") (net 1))
 (segment (start 186.49 114.92) (end 167.44 114.92) (width 0.2) (layer "B.Cu") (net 1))
 (segment (start 189.599999 94.352842) (end 186.49 97.462841) (width 0.2) (layer "B.Cu") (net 1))
 (segment (start 168 56.359999) (end 167.600001 55.96) (width 0.2) (layer "B.Cu") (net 1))
 (segment (start 165.2 58.849) (end 165.071 58.849) (width 0.2) (layer "F.Cu") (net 7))
 (segment (start 174.649 58.849) (end 165.2 58.849) (width 0.2) (layer "F.Cu") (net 7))
 (segment (start 165.2 58.849) (end 141.739 58.849) (width 0.2) (layer "F.Cu") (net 7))
 (segment (start 165.071 58.849) (end 163.92 60) (width 0.2) (layer "F.Cu") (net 7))
 (segment (start 141.739 58.849) (end 140 57.11) (width 0.2) (layer "F.Cu") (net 7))
 (segment (start 174.8 59) (end 174.649 58.849) (width 0.2) (layer "F.Cu") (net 7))
 (via (at 174.8 59) (size 0.6) (drill 0.3) (layers "F.Cu" "B.Cu") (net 7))
 (segment (start 177.835 58.165) (end 178 58) (width 0.2) (layer "B.Cu") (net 7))
 (segment (start 177.153 59) (end 174.8 59) (width 0.2) (layer "B.Cu") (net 7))
 (segment (start 177.835 58.318) (end 177.153 59) (width 0.2) (layer "B.Cu") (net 7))
 (segment (start 195.600001 94.147158) (end 195.689915 94.147158) (width 0.2) (layer "B.Cu") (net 13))
 (segment (start 139.52324 61.039) (end 138.849 61.71324) (width 0.2) (layer "B.Cu") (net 4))
 (segment (start 139.600001 94.147158) (end 139.600001 91.600001) (width 0.2) (layer "B.Cu") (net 4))
 (segment (start 140.47676 61.039) (end 139.52324 61.039) (width 0.2) (layer "B.Cu") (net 4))
 (segment (start 138.849 90.849) (end 139.600001 91.600001) (width 0.2) (layer "B.Cu") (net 4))
 (segment (start 138.849 61.71324) (end 138.849 90.849) (width 0.2) (layer "B.Cu") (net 4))
 (segment (start 145.55576 55.96) (end 140.47676 61.039) (width 0.2) (layer "B.Cu") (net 4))
 (segment (start 162.400001 55.96) (end 145.55576 55.96) (width 0.2) (layer "B.Cu") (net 4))
 (segment (start 162.399998 136.105684) (end 158.620868 136.105684) (width 0.2) (layer "B.Cu") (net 12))
 (segment (start 134.400001 111.884817) (end 134.400001 95.647158) (width 0.2) (layer "B.Cu") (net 12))
 (segment (start 158.620868 136.105684) (end 134.400001 111.884817) (width 0.2) (layer "B.Cu") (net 12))
 (segment (start 172.394316 134.605684) (end 167.599998 134.605684) (width 0.2) (layer "B.Cu") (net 11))
 (segment (start 190.399999 124.600001) (end 188 127) (width 0.2) (layer "B.Cu") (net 11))
 (segment (start 190.399999 95.852842) (end 190.399999 124.600001) (width 0.2) (layer "B.Cu") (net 11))
 (segment (start 180 127) (end 172.394316 134.605684) (width 0.2) (layer "B.Cu") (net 11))
 (segment (start 188 127) (end 180 127) (width 0.2) (layer "B.Cu") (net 11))
 (segment (start 132 126) (end 140.4 134.4) (width 0.2) (layer "B.Cu") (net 3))
 (segment (start 173 52) (end 174.238 53.238) (width 0.2) (layer "B.Cu") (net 3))
 (segment (start 174.238 53.238) (end 177.835 53.238) (width 0.2) (layer "B.Cu") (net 3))
 (segment (start 167.599998 136.105684) (end 172.105684 136.105684) (width 0.2) (layer "B.Cu") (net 3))
 (segment (start 163 52) (end 135 52) (width 0.2) (layer "B.Cu") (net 3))
 (segment (start 132 91.747157) (end 132 126) (width 0.2) (layer "B.Cu") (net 3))
 (segment (start 135 52) (end 132 55) (width 0.2) (layer "B.Cu") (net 3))
 (segment (start 195.599999 119.967101) (end 195.599999 95.852842) (width 0.2) (layer "B.Cu") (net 3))
 (segment (start 140.4 134.4) (end 155.4 134.4) (width 0.2) (layer "B.Cu") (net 3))
 (segment (start 162.400001 54.46) (end 162.400001 52.599999) (width 0.2) (layer "B.Cu") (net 3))
 (segment (start 170 139) (end 172.5 136.5) (width 0.2) (layer "B.Cu") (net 3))
 (segment (start 179.400001 129.599999) (end 172.5 136.5) (width 0.2) (layer "B.Cu") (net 3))
 (segment (start 132 91.747157) (end 134.400001 94.147158) (width 0.2) (layer "B.Cu") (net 3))
 (segment (start 132 55) (end 132 91.747157) (width 0.2) (layer "B.Cu") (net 3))
 (segment (start 155.4 134.4) (end 160 139) (width 0.2) (layer "B.Cu") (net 3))
 (segment (start 160 139) (end 170 139) (width 0.2) (layer "B.Cu") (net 3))
 (segment (start 185.967101 129.599999) (end 195.599999 119.967101) (width 0.2) (layer "B.Cu") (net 3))
 (segment (start 172.105684 136.105684) (end 172.5 136.5) (width 0.2) (layer "B.Cu") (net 3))
 (segment (start 162.400001 52.599999) (end 163 52) (width 0.2) (layer "B.Cu") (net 3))
 (segment (start 163 52) (end 173 52) (width 0.2) (layer "B.Cu") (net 3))
 (segment (start 179.400001 129.599999) (end 185.967101 129.599999) (width 0.2) (layer "B.Cu") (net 3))
 (segment (start 168.400001 54.46) (end 167.600001 54.46) (width 0.2) (layer "B.Cu") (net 5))
 (segment (start 167.973465 54.74355) (end 167.883551 54.74355) (width 0.2) (layer "B.Cu") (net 5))
 (segment (start 176.620942 69.779) (end 170.151 63.309058) (width 0.2) (layer "B.Cu") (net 5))
 (segment (start 179.049058 69.779) (end 176.620942 69.779) (width 0.2) (layer "B.Cu") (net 5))
 (segment (start 187.970058 60.858) (end 179.049058 69.779) (width 0.2) (layer "B.Cu") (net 5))
 (segment (start 170.151 56.210999) (end 168.400001 54.46) (width 0.2) (layer "B.Cu") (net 5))
 (segment (start 170.151 63.309058) (end 170.151 56.210999) (width 0.2) (layer "B.Cu") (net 5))
 (segment (start 194 60.858) (end 187.970058 60.858) (width 0.2) (layer "B.Cu") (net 5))
 (segment (start 181.793794 70.18) (end 175.437919 70.18) (width 0.2) (layer "B.Cu") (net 8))
 (segment (start 164.27 62.19) (end 164.83 61.63) (width 0.2) (layer "B.Cu") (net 8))
 (segment (start 175.437919 70.18) (end 166.46 61.202081) (width 0.2) (layer "B.Cu") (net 8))
 (segment (start 140 62.19) (end 164.27 62.19) (width 0.2) (layer "B.Cu") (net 8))
 (segment (start 164.83 61.63) (end 166.17645 60.28355) (width 0.2) (layer "B.Cu") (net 8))
 (segment (start 186.035794 65.938) (end 181.793794 70.18) (width 0.2) (layer "B.Cu") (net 8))
 (segment (start 194 65.938) (end 186.035794 65.938) (width 0.2) (layer "B.Cu") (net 8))
 (segment (start 166.46 61.202081) (end 166.46 60) (width 0.2) (layer "B.Cu") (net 8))
 (segment (start 164.27 64.73) (end 140 64.73) (width 0.2) (layer "F.Cu") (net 9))
 (segment (start 169 60) (end 164.27 64.73) (width 0.2) (layer "F.Cu") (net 9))
 (via (at 164.27 64.73) (size 0.6) (drill 0.3) (layers "F.Cu" "B.Cu") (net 9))
 (segment (start 194 63.398) (end 195.676 65.074) (width 0.2) (layer "B.Cu") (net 9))
 (segment (start 195.676 65.074) (end 195.676 69.317058) (width 0.2) (layer "B.Cu") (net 9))
 (segment (start 195.676 69.317058) (end 193.944058 71.049) (width 0.2) (layer "B.Cu") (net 9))
 (segment (start 193.944058 71.049) (end 170.589 71.049) (width 0.2) (layer "B.Cu") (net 9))
 (segment (start 170.589 71.049) (end 164.27 64.73) (width 0.2) (layer "B.Cu") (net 9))
 (segment (start 151 109) (end 150.49 109) (width 0.2) (layer "F.Cu") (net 2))
 (segment (start 150.49 109) (end 142.03 117.46) (width 0.2) (layer "F.Cu") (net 2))
 (via (at 151 109) (size 0.6) (drill 0.3) (layers "F.Cu" "B.Cu") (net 2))
 (segment (start 196.879 56.117) (end 196.879 78.538043) (width 0.2) (layer "B.Cu") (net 2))
 (segment (start 194 53.238) (end 196.879 56.117) (width 0.2) (layer "B.Cu") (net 2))
 (segment (start 196.879 78.538043) (end 166.417043 109) (width 0.2) (layer "B.Cu") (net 2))
 (segment (start 166.417043 109) (end 151 109) (width 0.2) (layer "B.Cu") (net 2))
 (segment (start 161 104) (end 161.09 104.09) (width 0.2) (layer "F.Cu") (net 10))
 (segment (start 161.09 104.09) (end 161.09 117.46) (width 0.2) (layer "F.Cu") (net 10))
 (segment (start 161 103) (end 161 104) (width 0.2) (layer "F.Cu") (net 10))
 (via (at 161 103) (size 0.6) (drill 0.3) (layers "F.Cu" "B.Cu") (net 10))
 (segment (start 196.478 58.256) (end 196.478 78.371943) (width 0.2) (layer "B.Cu") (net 10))
 (segment (start 171.849943 103) (end 161 103) (width 0.2) (layer "B.Cu") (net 10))
 (segment (start 194 55.778) (end 196.478 58.256) (width 0.2) (layer "B.Cu") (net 10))
 (segment (start 196.478 78.371943) (end 171.849943 103) (width 0.2) (layer "B.Cu") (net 10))
 (segment (start 180.14 94.86) (end 180.14 117.46) (width 0.2) (layer "F.Cu") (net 6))
 (segment (start 181 93) (end 181 94) (width 0.2) (layer "F.Cu") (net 6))
 (segment (start 181 94) (end 180.14 94.86) (width 0.2) (layer "F.Cu") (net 6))
 (via (at 181 93) (size 0.6) (drill 0.3) (layers "F.Cu" "B.Cu") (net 6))
 (segment (start 194 58.318) (end 196.077 60.395) (width 0.2) (layer "B.Cu") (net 6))
 (segment (start 196.077 60.395) (end 196.077 77.923) (width 0.2) (layer "B.Cu") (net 6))
 (segment (start 196.077 77.923) (end 181 93) (width 0.2) (layer "B.Cu") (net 6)))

